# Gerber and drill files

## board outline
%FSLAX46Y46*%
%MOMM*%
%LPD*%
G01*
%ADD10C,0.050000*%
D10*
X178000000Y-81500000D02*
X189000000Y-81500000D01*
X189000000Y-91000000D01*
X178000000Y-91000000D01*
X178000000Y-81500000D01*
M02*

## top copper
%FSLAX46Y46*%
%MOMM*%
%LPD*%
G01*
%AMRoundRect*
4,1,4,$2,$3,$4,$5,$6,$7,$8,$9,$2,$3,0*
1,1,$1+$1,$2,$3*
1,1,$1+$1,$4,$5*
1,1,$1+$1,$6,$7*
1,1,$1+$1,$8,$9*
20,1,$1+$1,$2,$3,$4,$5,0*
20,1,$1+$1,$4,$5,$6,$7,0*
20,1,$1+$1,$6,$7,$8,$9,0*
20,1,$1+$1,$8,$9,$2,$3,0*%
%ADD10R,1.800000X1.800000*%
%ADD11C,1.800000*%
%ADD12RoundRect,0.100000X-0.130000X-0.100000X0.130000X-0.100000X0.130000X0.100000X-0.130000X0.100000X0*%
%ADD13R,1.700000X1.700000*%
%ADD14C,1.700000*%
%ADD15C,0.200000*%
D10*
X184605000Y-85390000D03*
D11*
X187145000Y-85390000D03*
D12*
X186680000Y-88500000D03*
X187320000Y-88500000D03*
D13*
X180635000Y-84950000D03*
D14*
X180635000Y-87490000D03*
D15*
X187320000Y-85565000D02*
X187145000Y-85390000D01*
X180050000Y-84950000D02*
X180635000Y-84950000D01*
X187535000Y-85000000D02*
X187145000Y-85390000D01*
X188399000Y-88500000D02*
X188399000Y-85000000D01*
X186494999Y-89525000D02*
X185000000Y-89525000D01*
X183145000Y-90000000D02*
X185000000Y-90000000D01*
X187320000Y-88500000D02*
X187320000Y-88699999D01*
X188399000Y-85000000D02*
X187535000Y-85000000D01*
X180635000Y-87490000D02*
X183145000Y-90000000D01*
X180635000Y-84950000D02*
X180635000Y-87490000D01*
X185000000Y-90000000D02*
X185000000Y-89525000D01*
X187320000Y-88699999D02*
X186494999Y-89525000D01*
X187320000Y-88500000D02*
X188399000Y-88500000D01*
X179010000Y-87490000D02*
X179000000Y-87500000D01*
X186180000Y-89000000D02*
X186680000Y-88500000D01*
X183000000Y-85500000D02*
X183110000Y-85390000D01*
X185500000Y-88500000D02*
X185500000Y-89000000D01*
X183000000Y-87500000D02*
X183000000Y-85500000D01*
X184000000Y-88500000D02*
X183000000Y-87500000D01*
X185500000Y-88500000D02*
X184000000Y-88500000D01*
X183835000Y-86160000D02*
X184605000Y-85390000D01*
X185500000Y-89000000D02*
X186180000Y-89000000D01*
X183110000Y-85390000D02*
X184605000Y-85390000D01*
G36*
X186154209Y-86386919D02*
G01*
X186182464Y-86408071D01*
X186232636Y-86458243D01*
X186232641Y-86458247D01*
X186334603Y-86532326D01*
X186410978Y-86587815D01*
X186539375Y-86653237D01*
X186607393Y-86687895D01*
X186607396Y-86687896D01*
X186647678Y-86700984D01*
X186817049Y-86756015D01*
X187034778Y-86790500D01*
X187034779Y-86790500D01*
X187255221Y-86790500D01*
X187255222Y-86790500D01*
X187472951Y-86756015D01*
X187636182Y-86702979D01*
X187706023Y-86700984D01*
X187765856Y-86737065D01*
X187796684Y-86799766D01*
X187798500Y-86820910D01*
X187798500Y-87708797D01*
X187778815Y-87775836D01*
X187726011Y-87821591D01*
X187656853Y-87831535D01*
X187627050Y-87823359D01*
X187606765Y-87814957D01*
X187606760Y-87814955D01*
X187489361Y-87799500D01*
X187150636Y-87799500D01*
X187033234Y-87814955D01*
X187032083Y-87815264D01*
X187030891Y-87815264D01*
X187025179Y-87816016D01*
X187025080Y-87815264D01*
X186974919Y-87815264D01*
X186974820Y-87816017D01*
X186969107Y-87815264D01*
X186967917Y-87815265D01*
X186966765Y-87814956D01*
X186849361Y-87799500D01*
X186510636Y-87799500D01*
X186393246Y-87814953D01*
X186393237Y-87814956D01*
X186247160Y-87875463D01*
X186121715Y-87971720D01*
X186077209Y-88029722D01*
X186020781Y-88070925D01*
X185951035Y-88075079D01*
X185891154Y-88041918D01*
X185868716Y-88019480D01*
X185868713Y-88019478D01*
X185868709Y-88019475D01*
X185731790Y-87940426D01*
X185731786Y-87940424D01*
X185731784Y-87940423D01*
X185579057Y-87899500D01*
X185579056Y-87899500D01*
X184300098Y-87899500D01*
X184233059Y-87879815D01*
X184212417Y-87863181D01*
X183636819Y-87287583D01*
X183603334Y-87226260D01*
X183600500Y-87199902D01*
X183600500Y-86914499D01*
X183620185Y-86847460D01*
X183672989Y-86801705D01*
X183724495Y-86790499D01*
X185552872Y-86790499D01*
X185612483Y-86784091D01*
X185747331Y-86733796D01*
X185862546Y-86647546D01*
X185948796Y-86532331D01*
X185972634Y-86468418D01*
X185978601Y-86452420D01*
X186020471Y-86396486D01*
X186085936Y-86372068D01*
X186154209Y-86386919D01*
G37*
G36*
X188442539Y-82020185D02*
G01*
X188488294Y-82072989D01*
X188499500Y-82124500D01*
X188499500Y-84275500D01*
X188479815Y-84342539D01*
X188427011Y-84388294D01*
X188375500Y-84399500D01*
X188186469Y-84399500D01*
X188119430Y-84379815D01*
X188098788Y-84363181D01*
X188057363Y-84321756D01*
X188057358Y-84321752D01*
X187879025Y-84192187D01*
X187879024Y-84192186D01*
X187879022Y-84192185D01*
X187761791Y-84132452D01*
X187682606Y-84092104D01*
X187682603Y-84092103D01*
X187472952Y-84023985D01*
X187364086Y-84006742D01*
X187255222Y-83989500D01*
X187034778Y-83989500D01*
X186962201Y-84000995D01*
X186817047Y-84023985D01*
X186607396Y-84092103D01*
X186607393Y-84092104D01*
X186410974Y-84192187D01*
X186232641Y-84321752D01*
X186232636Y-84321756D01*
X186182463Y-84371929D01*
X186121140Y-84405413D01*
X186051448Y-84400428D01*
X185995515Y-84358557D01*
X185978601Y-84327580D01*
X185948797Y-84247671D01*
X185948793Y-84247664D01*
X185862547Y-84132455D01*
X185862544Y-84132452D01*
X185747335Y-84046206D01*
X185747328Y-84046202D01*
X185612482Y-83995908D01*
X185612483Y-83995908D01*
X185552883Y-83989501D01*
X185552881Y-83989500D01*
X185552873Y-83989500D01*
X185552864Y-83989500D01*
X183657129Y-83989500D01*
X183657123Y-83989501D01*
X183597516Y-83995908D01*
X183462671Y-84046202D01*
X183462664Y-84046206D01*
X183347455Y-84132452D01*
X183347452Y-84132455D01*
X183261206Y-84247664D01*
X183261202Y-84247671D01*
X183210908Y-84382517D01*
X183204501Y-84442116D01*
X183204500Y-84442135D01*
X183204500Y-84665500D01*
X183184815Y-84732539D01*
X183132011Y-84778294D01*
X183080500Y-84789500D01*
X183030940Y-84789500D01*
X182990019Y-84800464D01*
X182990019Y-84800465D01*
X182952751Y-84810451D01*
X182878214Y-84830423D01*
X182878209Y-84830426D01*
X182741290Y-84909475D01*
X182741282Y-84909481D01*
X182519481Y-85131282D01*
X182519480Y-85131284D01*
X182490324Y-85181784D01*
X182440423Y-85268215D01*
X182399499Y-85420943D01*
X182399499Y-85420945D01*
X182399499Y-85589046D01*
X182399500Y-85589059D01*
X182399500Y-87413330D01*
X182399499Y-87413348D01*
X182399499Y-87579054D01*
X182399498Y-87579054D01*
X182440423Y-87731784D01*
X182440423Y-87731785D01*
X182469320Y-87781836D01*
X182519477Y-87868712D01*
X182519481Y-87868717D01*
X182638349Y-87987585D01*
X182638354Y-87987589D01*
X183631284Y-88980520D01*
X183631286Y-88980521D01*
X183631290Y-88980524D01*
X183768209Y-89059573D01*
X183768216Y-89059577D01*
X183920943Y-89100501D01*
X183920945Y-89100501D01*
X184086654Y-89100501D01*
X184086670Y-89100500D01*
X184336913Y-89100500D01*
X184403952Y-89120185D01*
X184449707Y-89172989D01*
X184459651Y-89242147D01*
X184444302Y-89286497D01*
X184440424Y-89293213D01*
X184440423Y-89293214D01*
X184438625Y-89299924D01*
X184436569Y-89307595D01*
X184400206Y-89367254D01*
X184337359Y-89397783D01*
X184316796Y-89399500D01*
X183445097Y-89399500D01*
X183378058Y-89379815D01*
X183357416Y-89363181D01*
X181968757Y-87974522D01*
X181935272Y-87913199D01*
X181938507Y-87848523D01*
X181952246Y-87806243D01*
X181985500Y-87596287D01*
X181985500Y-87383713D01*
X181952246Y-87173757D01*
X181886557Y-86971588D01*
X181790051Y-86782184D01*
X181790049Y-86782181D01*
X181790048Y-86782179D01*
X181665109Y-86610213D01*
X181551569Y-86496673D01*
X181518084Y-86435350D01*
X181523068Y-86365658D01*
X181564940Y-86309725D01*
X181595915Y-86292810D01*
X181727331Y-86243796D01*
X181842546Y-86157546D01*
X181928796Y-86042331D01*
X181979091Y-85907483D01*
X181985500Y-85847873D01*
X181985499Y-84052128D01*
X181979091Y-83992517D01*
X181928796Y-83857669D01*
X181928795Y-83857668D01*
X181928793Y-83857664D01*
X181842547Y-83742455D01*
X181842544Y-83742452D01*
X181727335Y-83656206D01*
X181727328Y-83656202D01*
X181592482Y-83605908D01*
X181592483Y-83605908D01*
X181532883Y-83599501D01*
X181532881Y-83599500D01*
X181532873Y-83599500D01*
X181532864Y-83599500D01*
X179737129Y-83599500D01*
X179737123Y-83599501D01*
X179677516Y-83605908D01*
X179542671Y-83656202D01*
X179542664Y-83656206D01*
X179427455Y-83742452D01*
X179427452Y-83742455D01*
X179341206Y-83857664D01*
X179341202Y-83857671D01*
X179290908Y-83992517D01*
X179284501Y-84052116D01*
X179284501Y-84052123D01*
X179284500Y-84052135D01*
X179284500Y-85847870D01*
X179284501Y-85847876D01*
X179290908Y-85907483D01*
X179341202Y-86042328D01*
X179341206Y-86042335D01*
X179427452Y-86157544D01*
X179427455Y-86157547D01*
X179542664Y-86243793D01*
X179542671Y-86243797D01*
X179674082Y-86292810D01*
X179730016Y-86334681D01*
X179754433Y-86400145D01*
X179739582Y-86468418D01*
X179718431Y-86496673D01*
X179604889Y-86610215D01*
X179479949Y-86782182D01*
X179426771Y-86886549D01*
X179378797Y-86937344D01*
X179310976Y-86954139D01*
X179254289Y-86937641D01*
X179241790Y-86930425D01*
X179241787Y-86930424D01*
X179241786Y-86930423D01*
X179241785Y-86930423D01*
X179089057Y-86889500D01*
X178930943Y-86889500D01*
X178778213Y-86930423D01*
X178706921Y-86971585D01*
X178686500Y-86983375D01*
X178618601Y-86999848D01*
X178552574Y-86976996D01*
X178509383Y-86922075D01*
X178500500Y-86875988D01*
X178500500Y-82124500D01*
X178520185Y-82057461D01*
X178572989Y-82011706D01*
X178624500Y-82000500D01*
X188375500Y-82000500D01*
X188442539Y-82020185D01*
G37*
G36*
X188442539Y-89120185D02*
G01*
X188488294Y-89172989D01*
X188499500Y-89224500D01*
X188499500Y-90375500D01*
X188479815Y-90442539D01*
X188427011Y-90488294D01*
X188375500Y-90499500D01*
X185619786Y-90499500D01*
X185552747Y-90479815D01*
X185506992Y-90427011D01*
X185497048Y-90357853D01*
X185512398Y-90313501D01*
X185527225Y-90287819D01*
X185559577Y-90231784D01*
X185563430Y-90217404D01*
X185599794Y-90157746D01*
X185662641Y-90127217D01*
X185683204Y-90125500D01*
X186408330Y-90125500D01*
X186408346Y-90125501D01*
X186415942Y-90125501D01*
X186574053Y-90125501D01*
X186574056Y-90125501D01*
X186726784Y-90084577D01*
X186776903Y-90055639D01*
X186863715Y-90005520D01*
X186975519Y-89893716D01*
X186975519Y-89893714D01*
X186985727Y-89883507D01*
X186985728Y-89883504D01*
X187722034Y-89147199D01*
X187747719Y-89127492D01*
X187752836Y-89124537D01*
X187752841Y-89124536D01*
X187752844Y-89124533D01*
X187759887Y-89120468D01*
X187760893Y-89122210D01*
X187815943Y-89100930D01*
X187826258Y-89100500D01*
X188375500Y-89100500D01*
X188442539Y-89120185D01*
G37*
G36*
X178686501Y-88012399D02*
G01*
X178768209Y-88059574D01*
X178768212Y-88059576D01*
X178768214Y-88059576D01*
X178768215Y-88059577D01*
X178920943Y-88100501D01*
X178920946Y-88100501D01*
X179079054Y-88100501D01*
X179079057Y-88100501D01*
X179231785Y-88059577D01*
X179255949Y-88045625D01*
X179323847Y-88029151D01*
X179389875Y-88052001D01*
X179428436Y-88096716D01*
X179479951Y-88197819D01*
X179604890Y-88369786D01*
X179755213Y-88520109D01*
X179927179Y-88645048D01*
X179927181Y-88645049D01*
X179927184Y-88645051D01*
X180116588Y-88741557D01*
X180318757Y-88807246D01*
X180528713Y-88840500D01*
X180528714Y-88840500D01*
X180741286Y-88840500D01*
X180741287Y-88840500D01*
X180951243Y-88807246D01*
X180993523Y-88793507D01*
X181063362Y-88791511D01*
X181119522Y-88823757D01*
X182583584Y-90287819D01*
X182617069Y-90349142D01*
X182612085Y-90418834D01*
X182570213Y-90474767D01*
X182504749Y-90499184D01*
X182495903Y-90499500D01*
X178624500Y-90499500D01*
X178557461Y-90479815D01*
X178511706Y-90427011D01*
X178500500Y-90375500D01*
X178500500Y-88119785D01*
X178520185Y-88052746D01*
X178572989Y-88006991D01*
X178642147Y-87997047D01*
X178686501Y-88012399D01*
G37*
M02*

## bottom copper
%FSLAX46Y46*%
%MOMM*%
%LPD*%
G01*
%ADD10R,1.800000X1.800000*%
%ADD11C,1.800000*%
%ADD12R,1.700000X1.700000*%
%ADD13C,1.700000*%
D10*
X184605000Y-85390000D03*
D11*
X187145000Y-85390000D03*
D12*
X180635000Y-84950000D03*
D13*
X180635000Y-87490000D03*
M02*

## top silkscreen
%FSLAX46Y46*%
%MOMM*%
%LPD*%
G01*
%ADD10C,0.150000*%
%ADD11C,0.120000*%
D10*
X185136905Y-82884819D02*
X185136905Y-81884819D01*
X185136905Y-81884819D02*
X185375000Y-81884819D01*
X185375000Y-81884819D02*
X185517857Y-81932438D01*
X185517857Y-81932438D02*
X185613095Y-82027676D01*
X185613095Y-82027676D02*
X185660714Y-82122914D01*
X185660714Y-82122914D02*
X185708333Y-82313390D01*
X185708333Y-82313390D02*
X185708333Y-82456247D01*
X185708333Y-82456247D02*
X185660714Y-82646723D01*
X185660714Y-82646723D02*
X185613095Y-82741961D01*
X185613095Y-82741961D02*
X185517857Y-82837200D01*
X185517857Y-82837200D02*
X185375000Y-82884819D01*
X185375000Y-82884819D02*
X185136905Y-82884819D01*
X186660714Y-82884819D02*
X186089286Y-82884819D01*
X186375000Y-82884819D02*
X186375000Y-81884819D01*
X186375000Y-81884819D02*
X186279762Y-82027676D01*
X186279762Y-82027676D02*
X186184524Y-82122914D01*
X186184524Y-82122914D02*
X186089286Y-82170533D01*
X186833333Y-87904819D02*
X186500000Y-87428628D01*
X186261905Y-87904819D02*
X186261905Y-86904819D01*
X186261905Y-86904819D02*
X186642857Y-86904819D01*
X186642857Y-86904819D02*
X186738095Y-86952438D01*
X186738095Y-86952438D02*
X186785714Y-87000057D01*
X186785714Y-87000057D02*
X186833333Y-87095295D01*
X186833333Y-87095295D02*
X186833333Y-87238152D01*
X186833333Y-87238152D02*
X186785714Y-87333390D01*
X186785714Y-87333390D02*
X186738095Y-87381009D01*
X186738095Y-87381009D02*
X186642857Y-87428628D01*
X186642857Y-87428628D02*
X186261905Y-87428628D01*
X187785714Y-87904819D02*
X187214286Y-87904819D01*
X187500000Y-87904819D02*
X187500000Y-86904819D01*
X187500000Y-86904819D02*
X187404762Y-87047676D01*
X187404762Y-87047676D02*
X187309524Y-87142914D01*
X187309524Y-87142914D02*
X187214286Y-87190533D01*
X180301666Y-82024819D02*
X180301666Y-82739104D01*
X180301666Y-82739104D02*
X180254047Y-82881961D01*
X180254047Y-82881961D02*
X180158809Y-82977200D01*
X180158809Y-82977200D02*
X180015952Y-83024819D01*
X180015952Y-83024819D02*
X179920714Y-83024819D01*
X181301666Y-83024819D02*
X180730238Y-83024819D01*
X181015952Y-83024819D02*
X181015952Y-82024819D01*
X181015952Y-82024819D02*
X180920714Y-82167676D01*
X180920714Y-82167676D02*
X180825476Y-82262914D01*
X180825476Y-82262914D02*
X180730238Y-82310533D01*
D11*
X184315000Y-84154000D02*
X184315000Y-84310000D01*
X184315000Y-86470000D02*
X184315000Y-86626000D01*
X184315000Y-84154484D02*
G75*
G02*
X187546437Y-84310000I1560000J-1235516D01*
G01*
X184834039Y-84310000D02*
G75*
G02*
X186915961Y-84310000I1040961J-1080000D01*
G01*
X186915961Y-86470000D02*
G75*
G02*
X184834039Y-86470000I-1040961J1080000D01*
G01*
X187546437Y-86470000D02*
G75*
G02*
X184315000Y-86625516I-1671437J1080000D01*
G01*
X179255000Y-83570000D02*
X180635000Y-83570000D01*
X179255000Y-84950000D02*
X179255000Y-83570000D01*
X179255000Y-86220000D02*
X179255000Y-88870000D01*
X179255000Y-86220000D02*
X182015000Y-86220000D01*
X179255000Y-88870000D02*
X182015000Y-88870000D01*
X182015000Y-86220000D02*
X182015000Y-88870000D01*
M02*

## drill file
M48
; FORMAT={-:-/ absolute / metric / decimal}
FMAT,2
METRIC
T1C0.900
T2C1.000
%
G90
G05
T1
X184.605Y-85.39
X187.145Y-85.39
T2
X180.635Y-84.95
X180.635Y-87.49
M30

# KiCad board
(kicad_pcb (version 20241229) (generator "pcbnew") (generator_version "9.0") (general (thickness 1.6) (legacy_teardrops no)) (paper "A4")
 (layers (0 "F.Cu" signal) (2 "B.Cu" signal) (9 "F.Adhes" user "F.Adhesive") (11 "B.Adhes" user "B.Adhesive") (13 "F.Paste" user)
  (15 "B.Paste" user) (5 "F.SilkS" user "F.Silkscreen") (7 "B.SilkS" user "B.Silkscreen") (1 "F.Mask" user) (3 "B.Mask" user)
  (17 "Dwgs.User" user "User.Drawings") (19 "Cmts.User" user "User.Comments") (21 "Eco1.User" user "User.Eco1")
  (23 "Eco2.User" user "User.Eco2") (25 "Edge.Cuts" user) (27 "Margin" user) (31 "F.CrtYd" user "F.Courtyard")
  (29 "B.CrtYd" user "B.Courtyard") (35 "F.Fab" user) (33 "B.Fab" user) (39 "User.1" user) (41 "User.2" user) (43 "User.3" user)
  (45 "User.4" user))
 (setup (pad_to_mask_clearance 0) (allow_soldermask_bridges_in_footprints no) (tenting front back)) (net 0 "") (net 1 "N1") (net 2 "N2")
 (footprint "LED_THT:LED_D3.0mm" (layer "F.Cu") (at 184.605 85.39)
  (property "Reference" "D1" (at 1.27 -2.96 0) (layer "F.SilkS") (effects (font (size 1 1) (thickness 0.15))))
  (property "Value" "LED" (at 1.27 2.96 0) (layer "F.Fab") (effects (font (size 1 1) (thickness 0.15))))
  (fp_line (start -0.29 -1.236) (end -0.29 -1.08) (stroke (width 0.12) (type solid)) (layer "F.SilkS"))
  (fp_line (start -0.29 1.08) (end -0.29 1.236) (stroke (width 0.12) (type solid)) (layer "F.SilkS"))
  (fp_arc (start -0.29 -1.235516) (mid 1.36566 -1.987699) (end 2.941437 -1.08) (stroke (width 0.12) (type solid)) (layer "F.SilkS"))
  (fp_arc (start 0.229039 -1.08) (mid 1.27 -1.5) (end 2.310961 -1.08) (stroke (width 0.12) (type solid)) (layer "F.SilkS"))
  (fp_arc (start 2.310961 1.08) (mid 1.27 1.5) (end 0.229039 1.08) (stroke (width 0.12) (type solid)) (layer "F.SilkS"))
  (fp_arc (start 2.941437 1.08) (mid 1.36566 1.987699) (end -0.29 1.235516) (stroke (width 0.12) (type solid)) (layer "F.SilkS"))
  (pad "1" thru_hole rect (at 0 0) (size 1.8 1.8) (drill 0.9) (layers "*.Cu" "*.Mask") (remove_unused_layers no) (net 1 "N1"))
  (pad "2" thru_hole circle (at 2.54 0) (size 1.8 1.8) (drill 0.9) (layers "*.Cu" "*.Mask") (remove_unused_layers no) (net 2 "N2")))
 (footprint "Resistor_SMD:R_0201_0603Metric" (layer "F.Cu") (at 187 88.5)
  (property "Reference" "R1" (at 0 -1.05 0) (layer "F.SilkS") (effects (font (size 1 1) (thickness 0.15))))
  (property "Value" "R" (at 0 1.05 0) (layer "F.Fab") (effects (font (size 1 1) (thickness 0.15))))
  (pad "" smd roundrect (at -0.345 0) (size 0.318 0.36) (layers "F.Paste") (roundrect_rratio 0.25))
  (pad "" smd roundrect (at 0.345 0) (size 0.318 0.36) (layers "F.Paste") (roundrect_rratio 0.25))
  (pad "1" smd roundrect (at -0.32 0) (size 0.46 0.4) (layers "F.Cu" "F.Mask") (roundrect_rratio 0.25) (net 1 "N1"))
  (pad "2" smd roundrect (at 0.32 0) (size 0.46 0.4) (layers "F.Cu" "F.Mask") (roundrect_rratio 0.25) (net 2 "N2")))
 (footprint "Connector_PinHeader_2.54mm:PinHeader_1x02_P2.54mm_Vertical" (layer "F.Cu") (at 180.635 84.95)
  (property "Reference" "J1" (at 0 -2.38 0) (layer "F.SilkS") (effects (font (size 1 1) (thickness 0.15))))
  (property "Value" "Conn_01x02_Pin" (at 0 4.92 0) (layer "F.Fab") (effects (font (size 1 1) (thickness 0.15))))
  (fp_line (start -1.38 -1.38) (end 0 -1.38) (stroke (width 0.12) (type solid)) (layer "F.SilkS"))
  (fp_line (start -1.38 0) (end -1.38 -1.38) (stroke (width 0.12) (type solid)) (layer "F.SilkS"))
  (fp_line (start -1.38 1.27) (end -1.38 3.92) (stroke (width 0.12) (type solid)) (layer "F.SilkS"))
  (fp_line (start -1.38 1.27) (end 1.38 1.27) (stroke (width 0.12) (type solid)) (layer "F.SilkS"))
  (fp_line (start -1.38 3.92) (end 1.38 3.92) (stroke (width 0.12) (type solid)) (layer "F.SilkS"))
  (fp_line (start 1.38 1.27) (end 1.38 3.92) (stroke (width 0.12) (type solid)) (layer "F.SilkS"))
  (pad "1" thru_hole rect (at 0 0) (size 1.7 1.7) (drill 1) (layers "*.Cu" "*.Mask") (remove_unused_layers no) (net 2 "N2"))
  (pad "2" thru_hole circle (at 0 2.54) (size 1.7 1.7) (drill 1) (layers "*.Cu" "*.Mask") (remove_unused_layers no) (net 2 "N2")))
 (gr_rect (start 178 81.5) (end 189 91) (stroke (width 0.05) (type default)) (fill no) (layer "Edge.Cuts"))
 (segment (start 187.32 85.565) (end 187.145 85.39) (width 0.2) (layer "F.Cu") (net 2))
 (segment (start 180.05 84.95) (end 180.635 84.95) (width 0.2) (layer "F.Cu") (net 2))
 (segment (start 187.535 85) (end 187.145 85.39) (width 0.2) (layer "F.Cu") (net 2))
 (segment (start 188.399 88.5) (end 188.399 85) (width 0.2) (layer "F.Cu") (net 2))
 (segment (start 186.494999 89.525) (end 185 89.525) (width 0.2) (layer "F.Cu") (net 2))
 (segment (start 183.145 90) (end 185 90) (width 0.2) (layer "F.Cu") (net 2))
 (segment (start 187.32 88.5) (end 187.32 88.699999) (width 0.2) (layer "F.Cu") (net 2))
 (segment (start 188.399 85) (end 187.535 85) (width 0.2) (layer "F.Cu") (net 2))
 (segment (start 180.635 87.49) (end 183.145 90) (width 0.2) (layer "F.Cu") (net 2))
 (segment (start 180.635 84.95) (end 180.635 87.49) (width 0.2) (layer "F.Cu") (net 2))
 (segment (start 185 90) (end 185 89.525) (width 0.2) (layer "F.Cu") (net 2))
 (segment (start 187.32 88.699999) (end 186.494999 89.525) (width 0.2) (layer "F.Cu") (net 2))
 (segment (start 187.32 88.5) (end 188.399 88.5) (width 0.2) (layer "F.Cu") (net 2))
 (segment (start 179.01 87.49) (end 179 87.5) (width 0.2) (layer "F.Cu") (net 2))
 (segment (start 186.18 89) (end 186.68 88.5) (width 0.2) (layer "F.Cu") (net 1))
 (segment (start 183 85.5) (end 183.11 85.39) (width 0.2) (layer "F.Cu") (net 1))
 (segment (start 185.5 88.5) (end 185.5 89) (width 0.2) (layer "F.Cu") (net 1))
 (segment (start 183 87.5) (end 183 85.5) (width 0.2) (layer "F.Cu") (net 1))
 (segment (start 184 88.5) (end 183 87.5) (width 0.2) (layer "F.Cu") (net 1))
 (segment (start 185.5 88.5) (end 184 88.5) (width 0.2) (layer "F.Cu") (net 1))
 (segment (start 183.835 86.16) (end 184.605 85.39) (width 0.2) (layer "F.Cu") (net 1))
 (segment (start 185.5 89) (end 186.18 89) (width 0.2) (layer "F.Cu") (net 1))
 (segment (start 183.11 85.39) (end 184.605 85.39) (width 0.2) (layer "F.Cu") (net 1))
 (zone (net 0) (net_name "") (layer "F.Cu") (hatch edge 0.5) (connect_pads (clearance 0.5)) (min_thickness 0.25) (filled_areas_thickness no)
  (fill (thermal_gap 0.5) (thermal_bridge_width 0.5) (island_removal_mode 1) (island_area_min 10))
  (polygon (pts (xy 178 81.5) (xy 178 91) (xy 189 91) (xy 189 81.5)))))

